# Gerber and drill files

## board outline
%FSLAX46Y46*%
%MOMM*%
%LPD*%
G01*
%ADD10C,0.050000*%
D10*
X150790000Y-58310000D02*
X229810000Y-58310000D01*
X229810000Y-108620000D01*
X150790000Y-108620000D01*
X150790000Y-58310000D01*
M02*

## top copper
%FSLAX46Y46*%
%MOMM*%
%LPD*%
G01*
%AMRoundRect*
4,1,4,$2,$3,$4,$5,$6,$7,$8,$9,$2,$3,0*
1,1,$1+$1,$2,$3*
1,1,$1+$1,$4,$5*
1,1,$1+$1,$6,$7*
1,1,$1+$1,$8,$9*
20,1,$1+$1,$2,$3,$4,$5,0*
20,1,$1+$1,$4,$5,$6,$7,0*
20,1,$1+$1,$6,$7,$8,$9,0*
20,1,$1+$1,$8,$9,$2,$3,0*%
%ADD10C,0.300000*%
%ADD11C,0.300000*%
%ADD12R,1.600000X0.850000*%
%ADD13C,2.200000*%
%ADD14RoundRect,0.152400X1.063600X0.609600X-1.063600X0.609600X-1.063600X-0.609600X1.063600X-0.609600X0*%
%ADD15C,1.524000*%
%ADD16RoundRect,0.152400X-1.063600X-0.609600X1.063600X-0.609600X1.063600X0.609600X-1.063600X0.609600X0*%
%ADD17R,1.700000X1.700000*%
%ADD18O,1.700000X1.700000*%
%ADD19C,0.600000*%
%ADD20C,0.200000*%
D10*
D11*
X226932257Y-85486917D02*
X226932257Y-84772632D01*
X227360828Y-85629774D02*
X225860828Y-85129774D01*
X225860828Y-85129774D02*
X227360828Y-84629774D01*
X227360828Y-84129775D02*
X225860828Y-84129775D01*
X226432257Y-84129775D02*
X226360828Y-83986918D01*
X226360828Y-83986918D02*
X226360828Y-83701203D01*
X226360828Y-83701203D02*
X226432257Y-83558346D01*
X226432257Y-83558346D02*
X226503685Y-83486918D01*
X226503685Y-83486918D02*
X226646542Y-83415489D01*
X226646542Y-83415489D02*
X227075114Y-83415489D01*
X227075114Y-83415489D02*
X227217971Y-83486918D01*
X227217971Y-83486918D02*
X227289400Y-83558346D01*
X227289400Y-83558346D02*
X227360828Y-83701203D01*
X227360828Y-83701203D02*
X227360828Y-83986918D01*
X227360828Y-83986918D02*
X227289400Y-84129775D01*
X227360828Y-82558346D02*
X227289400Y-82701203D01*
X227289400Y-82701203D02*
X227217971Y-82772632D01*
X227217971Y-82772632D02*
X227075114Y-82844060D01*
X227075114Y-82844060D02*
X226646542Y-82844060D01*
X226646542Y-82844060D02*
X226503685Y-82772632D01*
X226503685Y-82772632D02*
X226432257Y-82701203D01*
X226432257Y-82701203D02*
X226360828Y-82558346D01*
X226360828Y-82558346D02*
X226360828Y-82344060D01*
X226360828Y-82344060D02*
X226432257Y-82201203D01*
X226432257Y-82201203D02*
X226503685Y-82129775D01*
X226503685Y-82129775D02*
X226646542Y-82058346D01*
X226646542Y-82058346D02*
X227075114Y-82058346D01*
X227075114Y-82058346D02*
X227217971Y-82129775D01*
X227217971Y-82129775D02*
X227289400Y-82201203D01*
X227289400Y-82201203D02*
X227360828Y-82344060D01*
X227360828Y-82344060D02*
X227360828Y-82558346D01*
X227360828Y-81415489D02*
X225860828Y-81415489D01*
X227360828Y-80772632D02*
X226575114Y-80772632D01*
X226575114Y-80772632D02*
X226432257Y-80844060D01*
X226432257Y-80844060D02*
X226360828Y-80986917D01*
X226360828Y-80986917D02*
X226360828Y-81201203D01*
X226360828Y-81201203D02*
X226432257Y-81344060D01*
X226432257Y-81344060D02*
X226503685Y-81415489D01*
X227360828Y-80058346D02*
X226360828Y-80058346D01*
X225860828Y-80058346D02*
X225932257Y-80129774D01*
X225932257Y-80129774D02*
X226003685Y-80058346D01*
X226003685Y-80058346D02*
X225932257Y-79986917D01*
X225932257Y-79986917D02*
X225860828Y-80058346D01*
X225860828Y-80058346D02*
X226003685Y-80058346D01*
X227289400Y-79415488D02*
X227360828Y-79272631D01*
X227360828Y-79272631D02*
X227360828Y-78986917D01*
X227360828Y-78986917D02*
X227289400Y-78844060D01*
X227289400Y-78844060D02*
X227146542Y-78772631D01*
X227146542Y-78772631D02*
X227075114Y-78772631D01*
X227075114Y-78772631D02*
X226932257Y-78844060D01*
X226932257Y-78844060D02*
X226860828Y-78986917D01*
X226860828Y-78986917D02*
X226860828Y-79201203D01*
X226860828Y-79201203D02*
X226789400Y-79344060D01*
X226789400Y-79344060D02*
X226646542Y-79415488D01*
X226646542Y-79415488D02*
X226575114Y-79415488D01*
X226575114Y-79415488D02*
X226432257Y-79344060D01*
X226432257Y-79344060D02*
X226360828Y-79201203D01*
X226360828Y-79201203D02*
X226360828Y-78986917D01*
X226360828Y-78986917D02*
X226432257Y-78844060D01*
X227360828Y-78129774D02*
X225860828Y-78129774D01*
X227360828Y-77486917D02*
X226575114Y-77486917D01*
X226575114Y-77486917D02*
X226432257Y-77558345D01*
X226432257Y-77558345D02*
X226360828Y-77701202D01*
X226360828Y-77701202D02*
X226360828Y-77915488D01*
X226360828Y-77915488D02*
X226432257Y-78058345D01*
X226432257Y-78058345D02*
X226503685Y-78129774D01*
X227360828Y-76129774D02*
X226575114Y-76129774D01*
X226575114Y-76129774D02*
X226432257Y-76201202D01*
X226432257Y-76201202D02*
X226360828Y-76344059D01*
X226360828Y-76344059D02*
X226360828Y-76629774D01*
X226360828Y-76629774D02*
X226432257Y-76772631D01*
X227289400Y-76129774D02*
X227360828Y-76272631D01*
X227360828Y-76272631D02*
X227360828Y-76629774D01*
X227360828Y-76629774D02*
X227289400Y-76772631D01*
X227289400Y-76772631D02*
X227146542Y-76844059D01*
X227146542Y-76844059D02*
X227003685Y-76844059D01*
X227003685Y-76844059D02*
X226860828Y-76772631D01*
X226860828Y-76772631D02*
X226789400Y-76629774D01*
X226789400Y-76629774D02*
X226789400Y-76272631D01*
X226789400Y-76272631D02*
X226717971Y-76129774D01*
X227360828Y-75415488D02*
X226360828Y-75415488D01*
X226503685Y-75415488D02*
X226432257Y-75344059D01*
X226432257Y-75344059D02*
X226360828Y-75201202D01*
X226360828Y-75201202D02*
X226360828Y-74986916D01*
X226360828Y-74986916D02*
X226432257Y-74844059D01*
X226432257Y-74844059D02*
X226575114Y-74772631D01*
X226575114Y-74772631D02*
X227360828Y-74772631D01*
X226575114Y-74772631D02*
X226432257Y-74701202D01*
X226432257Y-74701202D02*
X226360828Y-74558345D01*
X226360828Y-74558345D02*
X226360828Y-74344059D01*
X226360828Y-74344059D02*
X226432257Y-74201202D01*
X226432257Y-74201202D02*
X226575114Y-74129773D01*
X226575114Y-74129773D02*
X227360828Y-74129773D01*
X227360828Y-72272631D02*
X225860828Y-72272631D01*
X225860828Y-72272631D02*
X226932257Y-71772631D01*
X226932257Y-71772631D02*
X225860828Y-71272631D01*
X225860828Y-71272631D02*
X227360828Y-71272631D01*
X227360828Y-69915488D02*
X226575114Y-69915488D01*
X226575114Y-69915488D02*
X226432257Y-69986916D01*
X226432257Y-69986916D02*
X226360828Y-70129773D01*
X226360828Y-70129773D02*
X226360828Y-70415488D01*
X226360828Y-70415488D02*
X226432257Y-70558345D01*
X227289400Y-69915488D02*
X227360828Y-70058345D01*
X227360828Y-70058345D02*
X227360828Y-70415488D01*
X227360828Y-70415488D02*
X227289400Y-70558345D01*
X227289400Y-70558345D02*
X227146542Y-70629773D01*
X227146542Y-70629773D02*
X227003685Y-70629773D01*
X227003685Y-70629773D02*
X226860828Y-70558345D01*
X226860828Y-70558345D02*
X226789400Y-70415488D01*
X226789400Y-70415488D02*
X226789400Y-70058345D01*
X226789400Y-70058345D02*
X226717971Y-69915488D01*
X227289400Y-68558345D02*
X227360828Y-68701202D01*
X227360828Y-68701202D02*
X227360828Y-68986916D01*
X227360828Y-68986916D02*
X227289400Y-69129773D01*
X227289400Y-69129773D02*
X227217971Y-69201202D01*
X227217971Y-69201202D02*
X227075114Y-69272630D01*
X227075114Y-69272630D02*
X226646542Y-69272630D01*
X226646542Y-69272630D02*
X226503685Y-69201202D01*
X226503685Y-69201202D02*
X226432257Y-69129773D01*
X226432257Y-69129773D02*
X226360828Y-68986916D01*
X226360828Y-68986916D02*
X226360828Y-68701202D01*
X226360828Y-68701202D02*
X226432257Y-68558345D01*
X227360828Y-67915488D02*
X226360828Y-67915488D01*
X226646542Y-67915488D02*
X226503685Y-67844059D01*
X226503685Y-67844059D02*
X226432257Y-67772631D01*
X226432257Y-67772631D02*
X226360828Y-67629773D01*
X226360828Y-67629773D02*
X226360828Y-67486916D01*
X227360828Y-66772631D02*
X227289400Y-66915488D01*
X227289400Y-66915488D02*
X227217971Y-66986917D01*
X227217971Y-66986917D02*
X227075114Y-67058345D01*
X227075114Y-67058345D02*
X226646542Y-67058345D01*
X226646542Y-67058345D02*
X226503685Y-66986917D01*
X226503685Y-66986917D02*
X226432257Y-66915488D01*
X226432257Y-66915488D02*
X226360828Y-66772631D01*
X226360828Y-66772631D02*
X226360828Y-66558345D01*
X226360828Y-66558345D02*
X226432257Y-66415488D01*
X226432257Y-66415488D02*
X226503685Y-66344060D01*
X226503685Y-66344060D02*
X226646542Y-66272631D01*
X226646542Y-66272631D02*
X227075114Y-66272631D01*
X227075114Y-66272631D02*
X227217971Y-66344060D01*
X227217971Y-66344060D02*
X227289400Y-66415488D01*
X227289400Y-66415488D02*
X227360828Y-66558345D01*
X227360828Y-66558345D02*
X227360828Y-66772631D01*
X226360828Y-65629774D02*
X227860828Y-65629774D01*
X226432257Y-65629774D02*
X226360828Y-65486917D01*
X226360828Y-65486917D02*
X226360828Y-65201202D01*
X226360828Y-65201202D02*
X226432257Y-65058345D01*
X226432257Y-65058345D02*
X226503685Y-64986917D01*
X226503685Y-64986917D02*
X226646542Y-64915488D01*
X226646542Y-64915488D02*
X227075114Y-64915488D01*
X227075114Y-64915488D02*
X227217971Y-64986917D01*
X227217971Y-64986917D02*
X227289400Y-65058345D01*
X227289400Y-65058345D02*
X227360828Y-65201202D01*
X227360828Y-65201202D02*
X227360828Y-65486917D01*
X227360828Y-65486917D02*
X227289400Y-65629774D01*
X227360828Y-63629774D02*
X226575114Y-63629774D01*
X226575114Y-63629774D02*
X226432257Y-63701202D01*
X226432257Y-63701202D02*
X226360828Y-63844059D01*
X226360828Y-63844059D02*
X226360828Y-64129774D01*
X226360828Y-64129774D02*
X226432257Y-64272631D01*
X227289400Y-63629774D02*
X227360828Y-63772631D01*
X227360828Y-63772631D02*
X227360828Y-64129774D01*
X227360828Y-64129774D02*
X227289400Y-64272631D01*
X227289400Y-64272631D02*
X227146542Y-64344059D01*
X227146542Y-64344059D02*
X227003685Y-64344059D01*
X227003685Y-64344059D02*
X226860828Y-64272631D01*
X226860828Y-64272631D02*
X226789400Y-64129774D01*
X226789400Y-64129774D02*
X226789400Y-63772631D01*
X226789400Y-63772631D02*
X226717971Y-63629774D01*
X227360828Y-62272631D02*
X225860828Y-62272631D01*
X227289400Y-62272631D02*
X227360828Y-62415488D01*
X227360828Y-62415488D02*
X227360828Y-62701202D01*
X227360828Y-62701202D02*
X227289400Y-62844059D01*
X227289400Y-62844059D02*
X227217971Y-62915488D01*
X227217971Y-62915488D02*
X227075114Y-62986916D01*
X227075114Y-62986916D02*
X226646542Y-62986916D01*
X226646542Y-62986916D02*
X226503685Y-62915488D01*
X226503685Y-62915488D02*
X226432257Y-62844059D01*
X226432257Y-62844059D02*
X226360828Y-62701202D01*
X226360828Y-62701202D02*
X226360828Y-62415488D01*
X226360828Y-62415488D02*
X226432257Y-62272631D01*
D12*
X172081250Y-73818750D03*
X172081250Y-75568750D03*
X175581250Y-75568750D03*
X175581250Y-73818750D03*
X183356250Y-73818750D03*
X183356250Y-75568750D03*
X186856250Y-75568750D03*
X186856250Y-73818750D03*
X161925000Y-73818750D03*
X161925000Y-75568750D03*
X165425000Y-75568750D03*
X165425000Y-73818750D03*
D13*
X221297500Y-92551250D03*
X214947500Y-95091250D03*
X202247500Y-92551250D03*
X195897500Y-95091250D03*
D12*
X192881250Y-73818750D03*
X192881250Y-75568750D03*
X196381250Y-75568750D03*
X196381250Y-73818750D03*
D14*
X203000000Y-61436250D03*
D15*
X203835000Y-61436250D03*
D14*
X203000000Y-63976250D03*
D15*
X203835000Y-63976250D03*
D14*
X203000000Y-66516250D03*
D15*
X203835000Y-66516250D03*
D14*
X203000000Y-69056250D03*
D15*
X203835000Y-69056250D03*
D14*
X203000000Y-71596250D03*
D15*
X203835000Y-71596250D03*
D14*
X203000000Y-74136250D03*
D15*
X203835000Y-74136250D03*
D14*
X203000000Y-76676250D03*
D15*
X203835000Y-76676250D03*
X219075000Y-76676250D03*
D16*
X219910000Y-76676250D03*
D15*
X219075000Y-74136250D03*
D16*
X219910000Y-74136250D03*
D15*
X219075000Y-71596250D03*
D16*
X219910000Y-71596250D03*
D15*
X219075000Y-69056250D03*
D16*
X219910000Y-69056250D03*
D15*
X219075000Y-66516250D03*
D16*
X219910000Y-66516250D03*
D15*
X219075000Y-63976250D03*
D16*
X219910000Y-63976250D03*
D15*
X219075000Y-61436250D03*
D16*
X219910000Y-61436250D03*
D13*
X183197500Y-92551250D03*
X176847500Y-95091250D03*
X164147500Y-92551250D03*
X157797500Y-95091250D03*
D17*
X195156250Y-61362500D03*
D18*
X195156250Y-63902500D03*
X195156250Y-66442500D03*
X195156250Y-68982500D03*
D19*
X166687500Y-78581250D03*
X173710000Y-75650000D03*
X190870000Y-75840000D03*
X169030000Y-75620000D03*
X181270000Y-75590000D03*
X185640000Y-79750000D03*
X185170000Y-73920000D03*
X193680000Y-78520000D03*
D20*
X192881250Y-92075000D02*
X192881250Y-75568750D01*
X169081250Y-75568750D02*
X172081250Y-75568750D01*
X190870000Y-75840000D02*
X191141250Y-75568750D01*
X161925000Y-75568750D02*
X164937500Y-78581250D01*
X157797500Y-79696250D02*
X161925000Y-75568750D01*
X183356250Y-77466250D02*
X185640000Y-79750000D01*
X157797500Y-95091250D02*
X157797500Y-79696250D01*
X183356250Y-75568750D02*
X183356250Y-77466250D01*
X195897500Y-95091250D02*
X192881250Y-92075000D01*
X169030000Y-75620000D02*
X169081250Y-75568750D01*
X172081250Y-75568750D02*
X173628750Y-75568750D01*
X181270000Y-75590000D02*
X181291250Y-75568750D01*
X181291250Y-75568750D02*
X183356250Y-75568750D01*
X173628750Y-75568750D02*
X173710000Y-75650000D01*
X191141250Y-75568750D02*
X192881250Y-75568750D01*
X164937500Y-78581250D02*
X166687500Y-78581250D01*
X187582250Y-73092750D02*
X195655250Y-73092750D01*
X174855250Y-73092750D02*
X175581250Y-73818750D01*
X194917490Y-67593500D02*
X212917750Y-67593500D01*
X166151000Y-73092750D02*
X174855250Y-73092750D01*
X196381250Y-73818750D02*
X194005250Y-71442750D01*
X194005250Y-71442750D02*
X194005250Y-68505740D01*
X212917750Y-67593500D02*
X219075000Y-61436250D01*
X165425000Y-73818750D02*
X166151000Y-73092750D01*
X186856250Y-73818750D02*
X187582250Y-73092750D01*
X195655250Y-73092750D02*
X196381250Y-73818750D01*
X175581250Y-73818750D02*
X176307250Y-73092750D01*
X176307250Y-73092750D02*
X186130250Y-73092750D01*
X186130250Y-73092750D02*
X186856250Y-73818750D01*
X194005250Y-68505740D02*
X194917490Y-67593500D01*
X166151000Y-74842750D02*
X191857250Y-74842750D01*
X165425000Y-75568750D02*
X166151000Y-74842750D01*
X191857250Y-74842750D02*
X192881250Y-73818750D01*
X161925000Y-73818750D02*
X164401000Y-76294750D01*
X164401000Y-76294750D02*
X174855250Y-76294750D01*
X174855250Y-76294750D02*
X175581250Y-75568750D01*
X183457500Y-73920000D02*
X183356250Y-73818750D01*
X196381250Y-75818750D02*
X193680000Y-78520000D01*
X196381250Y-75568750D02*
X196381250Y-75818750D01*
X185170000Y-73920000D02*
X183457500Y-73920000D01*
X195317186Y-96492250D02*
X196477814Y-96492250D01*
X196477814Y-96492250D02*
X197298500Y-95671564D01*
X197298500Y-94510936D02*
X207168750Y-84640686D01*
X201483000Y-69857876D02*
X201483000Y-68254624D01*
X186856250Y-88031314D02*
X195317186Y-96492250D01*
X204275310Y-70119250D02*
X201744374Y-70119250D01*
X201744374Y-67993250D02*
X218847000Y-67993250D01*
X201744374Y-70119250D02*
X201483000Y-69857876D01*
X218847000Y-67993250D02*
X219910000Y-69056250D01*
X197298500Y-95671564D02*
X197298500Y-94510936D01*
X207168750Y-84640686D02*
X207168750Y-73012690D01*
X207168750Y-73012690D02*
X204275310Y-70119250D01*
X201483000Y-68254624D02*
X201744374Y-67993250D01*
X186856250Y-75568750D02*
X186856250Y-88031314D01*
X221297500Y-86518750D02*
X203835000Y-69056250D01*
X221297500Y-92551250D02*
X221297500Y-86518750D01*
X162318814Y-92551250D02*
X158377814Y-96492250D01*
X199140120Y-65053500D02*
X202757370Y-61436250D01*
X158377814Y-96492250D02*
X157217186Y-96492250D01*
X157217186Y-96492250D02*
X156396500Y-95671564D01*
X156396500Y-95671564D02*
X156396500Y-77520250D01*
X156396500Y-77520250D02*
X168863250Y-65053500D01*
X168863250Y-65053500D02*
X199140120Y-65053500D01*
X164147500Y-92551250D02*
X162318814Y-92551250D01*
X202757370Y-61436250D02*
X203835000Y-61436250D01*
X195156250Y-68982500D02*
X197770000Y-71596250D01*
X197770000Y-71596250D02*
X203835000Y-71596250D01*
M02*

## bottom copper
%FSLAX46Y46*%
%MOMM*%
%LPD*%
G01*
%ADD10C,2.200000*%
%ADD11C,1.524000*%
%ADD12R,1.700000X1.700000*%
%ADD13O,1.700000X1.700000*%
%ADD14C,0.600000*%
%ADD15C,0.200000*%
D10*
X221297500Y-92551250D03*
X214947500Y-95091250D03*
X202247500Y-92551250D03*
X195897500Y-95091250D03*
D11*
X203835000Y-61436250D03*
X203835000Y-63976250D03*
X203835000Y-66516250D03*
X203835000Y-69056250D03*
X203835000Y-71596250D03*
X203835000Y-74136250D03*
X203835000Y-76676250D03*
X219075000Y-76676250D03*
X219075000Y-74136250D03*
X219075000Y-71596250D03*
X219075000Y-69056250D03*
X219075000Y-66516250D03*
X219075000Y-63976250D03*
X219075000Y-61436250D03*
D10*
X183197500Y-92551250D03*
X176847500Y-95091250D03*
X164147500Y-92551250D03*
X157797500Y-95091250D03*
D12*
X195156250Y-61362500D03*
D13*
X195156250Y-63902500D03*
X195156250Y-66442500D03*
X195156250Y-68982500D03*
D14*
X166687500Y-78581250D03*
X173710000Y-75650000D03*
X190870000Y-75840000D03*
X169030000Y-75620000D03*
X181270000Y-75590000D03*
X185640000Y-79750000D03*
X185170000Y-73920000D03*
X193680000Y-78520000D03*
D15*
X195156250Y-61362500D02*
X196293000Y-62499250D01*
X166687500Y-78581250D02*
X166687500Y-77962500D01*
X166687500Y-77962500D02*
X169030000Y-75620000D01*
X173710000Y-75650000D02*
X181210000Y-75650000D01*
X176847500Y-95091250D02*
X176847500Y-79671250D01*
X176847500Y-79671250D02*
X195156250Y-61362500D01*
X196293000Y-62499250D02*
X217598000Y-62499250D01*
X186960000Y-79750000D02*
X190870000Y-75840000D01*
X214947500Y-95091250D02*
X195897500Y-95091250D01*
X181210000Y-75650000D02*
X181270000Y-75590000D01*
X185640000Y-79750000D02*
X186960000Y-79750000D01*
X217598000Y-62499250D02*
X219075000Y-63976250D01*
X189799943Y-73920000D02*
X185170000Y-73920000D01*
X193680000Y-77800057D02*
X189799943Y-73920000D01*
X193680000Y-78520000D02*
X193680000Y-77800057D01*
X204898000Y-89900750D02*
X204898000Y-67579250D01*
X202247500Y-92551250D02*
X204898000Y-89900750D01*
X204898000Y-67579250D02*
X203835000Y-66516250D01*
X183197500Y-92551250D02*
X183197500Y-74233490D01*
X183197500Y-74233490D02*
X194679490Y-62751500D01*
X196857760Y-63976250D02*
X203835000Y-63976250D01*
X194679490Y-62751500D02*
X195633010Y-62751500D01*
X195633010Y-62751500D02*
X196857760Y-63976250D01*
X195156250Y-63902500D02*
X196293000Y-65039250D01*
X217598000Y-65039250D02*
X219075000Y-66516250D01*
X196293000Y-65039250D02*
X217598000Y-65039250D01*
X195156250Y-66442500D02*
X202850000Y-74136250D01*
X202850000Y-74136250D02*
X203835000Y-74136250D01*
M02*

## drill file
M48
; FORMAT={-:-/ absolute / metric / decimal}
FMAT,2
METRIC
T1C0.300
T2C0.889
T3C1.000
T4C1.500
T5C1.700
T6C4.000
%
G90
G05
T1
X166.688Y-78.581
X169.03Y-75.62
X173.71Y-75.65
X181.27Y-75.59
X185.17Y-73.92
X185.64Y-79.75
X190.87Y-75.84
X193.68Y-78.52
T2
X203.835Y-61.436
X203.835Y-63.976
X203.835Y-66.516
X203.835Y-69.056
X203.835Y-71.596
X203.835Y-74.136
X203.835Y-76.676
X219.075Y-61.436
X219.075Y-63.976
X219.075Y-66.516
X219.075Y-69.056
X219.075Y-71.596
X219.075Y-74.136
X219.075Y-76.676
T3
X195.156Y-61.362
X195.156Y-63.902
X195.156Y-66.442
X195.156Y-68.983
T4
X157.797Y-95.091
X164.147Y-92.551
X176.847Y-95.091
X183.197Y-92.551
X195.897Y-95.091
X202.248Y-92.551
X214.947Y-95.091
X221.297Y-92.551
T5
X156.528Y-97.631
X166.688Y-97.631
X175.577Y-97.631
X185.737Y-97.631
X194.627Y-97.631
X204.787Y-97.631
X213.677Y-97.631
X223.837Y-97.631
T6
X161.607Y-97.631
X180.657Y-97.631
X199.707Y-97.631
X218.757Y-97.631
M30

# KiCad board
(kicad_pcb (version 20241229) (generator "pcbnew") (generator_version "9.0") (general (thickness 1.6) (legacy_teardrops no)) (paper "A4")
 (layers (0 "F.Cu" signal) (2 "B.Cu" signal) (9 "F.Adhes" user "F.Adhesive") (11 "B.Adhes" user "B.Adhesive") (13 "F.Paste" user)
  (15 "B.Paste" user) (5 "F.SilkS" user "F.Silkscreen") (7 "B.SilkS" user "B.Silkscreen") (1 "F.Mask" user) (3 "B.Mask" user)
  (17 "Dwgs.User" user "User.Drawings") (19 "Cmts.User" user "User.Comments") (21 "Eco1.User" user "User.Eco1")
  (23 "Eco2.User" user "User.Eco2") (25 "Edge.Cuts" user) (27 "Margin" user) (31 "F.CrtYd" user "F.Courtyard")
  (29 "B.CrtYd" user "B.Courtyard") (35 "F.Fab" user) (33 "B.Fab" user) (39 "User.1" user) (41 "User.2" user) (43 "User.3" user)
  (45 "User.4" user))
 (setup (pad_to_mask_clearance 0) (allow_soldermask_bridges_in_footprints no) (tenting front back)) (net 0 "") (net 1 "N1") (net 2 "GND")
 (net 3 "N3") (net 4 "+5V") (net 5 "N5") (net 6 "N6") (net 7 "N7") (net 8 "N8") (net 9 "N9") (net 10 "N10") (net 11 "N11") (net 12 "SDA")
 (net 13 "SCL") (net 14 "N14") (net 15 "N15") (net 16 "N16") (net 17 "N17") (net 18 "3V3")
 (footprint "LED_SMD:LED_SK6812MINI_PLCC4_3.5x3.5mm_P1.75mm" (layer "F.Cu") (at 173.83125 74.69375)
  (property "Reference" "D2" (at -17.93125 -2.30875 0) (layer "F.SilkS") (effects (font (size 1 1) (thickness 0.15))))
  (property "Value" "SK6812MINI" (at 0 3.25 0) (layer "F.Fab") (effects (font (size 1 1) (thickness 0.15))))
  (pad "1" smd rect (at -1.75 -0.875) (size 1.6 0.85) (layers "F.Cu" "F.Mask" "F.Paste") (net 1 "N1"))
  (pad "2" smd rect (at -1.75 0.875) (size 1.6 0.85) (layers "F.Cu" "F.Mask" "F.Paste") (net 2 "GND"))
  (pad "3" smd rect (at 1.75 0.875) (size 1.6 0.85) (layers "F.Cu" "F.Mask" "F.Paste") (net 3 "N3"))
  (pad "4" smd rect (at 1.75 -0.875) (size 1.6 0.85) (layers "F.Cu" "F.Mask" "F.Paste") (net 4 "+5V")))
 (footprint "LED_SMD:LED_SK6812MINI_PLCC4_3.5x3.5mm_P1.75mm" (layer "F.Cu") (at 185.10625 74.69375)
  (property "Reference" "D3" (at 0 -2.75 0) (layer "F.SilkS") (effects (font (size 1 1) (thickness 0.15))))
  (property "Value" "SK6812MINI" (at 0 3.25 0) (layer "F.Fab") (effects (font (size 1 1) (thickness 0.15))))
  (pad "1" smd rect (at -1.75 -0.875) (size 1.6 0.85) (layers "F.Cu" "F.Mask" "F.Paste") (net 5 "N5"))
  (pad "2" smd rect (at -1.75 0.875) (size 1.6 0.85) (layers "F.Cu" "F.Mask" "F.Paste") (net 2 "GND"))
  (pad "3" smd rect (at 1.75 0.875) (size 1.6 0.85) (layers "F.Cu" "F.Mask" "F.Paste") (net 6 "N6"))
  (pad "4" smd rect (at 1.75 -0.875) (size 1.6 0.85) (layers "F.Cu" "F.Mask" "F.Paste") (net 4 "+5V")))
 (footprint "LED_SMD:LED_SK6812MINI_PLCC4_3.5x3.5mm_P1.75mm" (layer "F.Cu") (at 163.675 74.69375)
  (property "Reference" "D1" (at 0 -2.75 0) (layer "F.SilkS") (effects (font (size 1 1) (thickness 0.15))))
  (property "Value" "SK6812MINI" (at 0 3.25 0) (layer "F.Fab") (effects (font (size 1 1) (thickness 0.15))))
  (pad "1" smd rect (at -1.75 -0.875) (size 1.6 0.85) (layers "F.Cu" "F.Mask" "F.Paste") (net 3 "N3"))
  (pad "2" smd rect (at -1.75 0.875) (size 1.6 0.85) (layers "F.Cu" "F.Mask" "F.Paste") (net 2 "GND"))
  (pad "3" smd rect (at 1.75 0.875) (size 1.6 0.85) (layers "F.Cu" "F.Mask" "F.Paste") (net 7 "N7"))
  (pad "4" smd rect (at 1.75 -0.875) (size 1.6 0.85) (layers "F.Cu" "F.Mask" "F.Paste") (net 4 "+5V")))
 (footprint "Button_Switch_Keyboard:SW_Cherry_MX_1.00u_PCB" (layer "F.Cu") (at 221.2975 92.55125)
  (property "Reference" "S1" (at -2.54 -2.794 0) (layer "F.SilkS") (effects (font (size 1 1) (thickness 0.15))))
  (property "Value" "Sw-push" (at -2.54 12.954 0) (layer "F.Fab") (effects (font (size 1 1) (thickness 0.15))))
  (pad "" np_thru_hole circle (at -7.62 5.08) (size 1.7 1.7) (drill 1.7) (layers "*.Cu" "*.Mask"))
  (pad "" np_thru_hole circle (at -2.54 5.08) (size 4 4) (drill 4) (layers "*.Cu" "*.Mask"))
  (pad "" np_thru_hole circle (at 2.54 5.08) (size 1.7 1.7) (drill 1.7) (layers "*.Cu" "*.Mask"))
  (pad "1" thru_hole circle (at 0 0) (size 2.2 2.2) (drill 1.5) (layers "*.Cu" "*.Mask") (remove_unused_layers no) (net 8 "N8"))
  (pad "2" thru_hole circle (at -6.35 2.54) (size 2.2 2.2) (drill 1.5) (layers "*.Cu" "*.Mask") (remove_unused_layers no) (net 2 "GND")))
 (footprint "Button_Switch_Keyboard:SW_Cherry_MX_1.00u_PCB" (layer "F.Cu") (at 202.2475 92.55125)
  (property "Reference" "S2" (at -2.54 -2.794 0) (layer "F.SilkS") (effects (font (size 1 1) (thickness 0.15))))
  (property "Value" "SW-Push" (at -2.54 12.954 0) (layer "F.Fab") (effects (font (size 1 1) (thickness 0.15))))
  (pad "" np_thru_hole circle (at -7.62 5.08) (size 1.7 1.7) (drill 1.7) (layers "*.Cu" "*.Mask"))
  (pad "" np_thru_hole circle (at -2.54 5.08) (size 4 4) (drill 4) (layers "*.Cu" "*.Mask"))
  (pad "" np_thru_hole circle (at 2.54 5.08) (size 1.7 1.7) (drill 1.7) (layers "*.Cu" "*.Mask"))
  (pad "1" thru_hole circle (at 0 0) (size 2.2 2.2) (drill 1.5) (layers "*.Cu" "*.Mask") (remove_unused_layers no) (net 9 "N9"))
  (pad "2" thru_hole circle (at -6.35 2.54) (size 2.2 2.2) (drill 1.5) (layers "*.Cu" "*.Mask") (remove_unused_layers no) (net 2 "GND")))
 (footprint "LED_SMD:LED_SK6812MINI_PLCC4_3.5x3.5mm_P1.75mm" (layer "F.Cu") (at 194.63125 74.69375)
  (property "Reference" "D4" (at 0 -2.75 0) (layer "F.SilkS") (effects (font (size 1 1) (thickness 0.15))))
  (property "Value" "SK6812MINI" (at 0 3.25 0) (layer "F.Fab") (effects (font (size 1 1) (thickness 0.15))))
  (pad "1" smd rect (at -1.75 -0.875) (size 1.6 0.85) (layers "F.Cu" "F.Mask" "F.Paste") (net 7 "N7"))
  (pad "2" smd rect (at -1.75 0.875) (size 1.6 0.85) (layers "F.Cu" "F.Mask" "F.Paste") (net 2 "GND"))
  (pad "3" smd rect (at 1.75 0.875) (size 1.6 0.85) (layers "F.Cu" "F.Mask" "F.Paste") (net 5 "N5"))
  (pad "4" smd rect (at 1.75 -0.875) (size 1.6 0.85) (layers "F.Cu" "F.Mask" "F.Paste") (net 4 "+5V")))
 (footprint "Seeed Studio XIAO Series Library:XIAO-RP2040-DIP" (layer "F.Cu") (at 211.455 69.05625)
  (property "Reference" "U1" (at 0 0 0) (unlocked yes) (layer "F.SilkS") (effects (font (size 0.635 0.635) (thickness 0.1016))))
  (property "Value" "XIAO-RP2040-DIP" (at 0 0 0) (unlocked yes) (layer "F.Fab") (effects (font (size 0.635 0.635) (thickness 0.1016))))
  (pad "1" smd roundrect (at -8.455 -7.62 180) (size 2.432 1.524) (layers "F.Cu" "F.Mask") (roundrect_rratio 0.1) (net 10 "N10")
   (thermal_bridge_angle 45))
  (pad "1" thru_hole circle (at -7.62 -7.62 180) (size 1.524 1.524) (drill 0.889) (layers "*.Cu" "*.Mask") (remove_unused_layers no)
   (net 10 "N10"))
  (pad "2" smd roundrect (at -8.455 -5.08 180) (size 2.432 1.524) (layers "F.Cu" "F.Mask") (roundrect_rratio 0.1) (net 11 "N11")
   (thermal_bridge_angle 45))
  (pad "2" thru_hole circle (at -7.62 -5.08 180) (size 1.524 1.524) (drill 0.889) (layers "*.Cu" "*.Mask") (remove_unused_layers no)
   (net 11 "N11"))
  (pad "3" smd roundrect (at -8.455 -2.54 180) (size 2.432 1.524) (layers "F.Cu" "F.Mask") (roundrect_rratio 0.1) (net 9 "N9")
   (thermal_bridge_angle 45))
  (pad "3" thru_hole circle (at -7.62 -2.54 180) (size 1.524 1.524) (drill 0.889) (layers "*.Cu" "*.Mask") (remove_unused_layers no)
   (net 9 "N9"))
  (pad "4" smd roundrect (at -8.455 0 180) (size 2.432 1.524) (layers "F.Cu" "F.Mask") (roundrect_rratio 0.1) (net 8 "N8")
   (thermal_bridge_angle 45))
  (pad "4" thru_hole circle (at -7.62 0 180) (size 1.524 1.524) (drill 0.889) (layers "*.Cu" "*.Mask") (remove_unused_layers no)
   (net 8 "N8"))
  (pad "5" smd roundrect (at -8.455 2.54 180) (size 2.432 1.524) (layers "F.Cu" "F.Mask") (roundrect_rratio 0.1) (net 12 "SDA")
   (thermal_bridge_angle 45))
  (pad "5" thru_hole circle (at -7.62 2.54 180) (size 1.524 1.524) (drill 0.889) (layers "*.Cu" "*.Mask") (remove_unused_layers no)
   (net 12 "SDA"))
  (pad "6" smd roundrect (at -8.455 5.08 180) (size 2.432 1.524) (layers "F.Cu" "F.Mask") (roundrect_rratio 0.1) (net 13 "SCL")
   (thermal_bridge_angle 45))
  (pad "6" thru_hole circle (at -7.62 5.08 180) (size 1.524 1.524) (drill 0.889) (layers "*.Cu" "*.Mask") (remove_unused_layers no)
   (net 13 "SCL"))
  (pad "7" smd roundrect (at -8.455 7.62 180) (size 2.432 1.524) (layers "F.Cu" "F.Mask") (roundrect_rratio 0.1) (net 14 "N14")
   (thermal_bridge_angle 45))
  (pad "7" thru_hole circle (at -7.62 7.62 180) (size 1.524 1.524) (drill 0.889) (layers "*.Cu" "*.Mask") (remove_unused_layers no)
   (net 14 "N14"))
  (pad "8" thru_hole circle (at 7.62 7.62) (size 1.524 1.524) (drill 0.889) (layers "*.Cu" "*.Mask") (remove_unused_layers no)
   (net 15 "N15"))
  (pad "8" smd roundrect (at 8.455 7.62) (size 2.432 1.524) (layers "F.Cu" "F.Mask") (roundrect_rratio 0.1) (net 15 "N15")
   (thermal_bridge_angle 45))
  (pad "9" thru_hole circle (at 7.62 5.08) (size 1.524 1.524) (drill 0.889) (layers "*.Cu" "*.Mask") (remove_unused_layers no)
   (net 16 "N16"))
  (pad "9" smd roundrect (at 8.455 5.08) (size 2.432 1.524) (layers "F.Cu" "F.Mask") (roundrect_rratio 0.1) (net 16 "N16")
   (thermal_bridge_angle 45))
  (pad "10" thru_hole circle (at 7.62 2.54) (size 1.524 1.524) (drill 0.889) (layers "*.Cu" "*.Mask") (remove_unused_layers no)
   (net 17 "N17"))
  (pad "10" smd roundrect (at 8.455 2.54) (size 2.432 1.524) (layers "F.Cu" "F.Mask") (roundrect_rratio 0.1) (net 17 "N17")
   (thermal_bridge_angle 45))
  (pad "11" thru_hole circle (at 7.62 0) (size 1.524 1.524) (drill 0.889) (layers "*.Cu" "*.Mask") (remove_unused_layers no) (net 6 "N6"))
  (pad "11" smd roundrect (at 8.455 0) (size 2.432 1.524) (layers "F.Cu" "F.Mask") (roundrect_rratio 0.1) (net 6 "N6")
   (thermal_bridge_angle 45))
  (pad "12" thru_hole circle (at 7.62 -2.54) (size 1.524 1.524) (drill 0.889) (layers "*.Cu" "*.Mask") (remove_unused_layers no)
   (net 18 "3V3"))
  (pad "12" smd roundrect (at 8.455 -2.54) (size 2.432 1.524) (layers "F.Cu" "F.Mask") (roundrect_rratio 0.1) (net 18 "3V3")
   (thermal_bridge_angle 45))
  (pad "13" thru_hole circle (at 7.62 -5.08) (size 1.524 1.524) (drill 0.889) (layers "*.Cu" "*.Mask") (remove_unused_layers no)
   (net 2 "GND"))
  (pad "13" smd roundrect (at 8.455 -5.08) (size 2.432 1.524) (layers "F.Cu" "F.Mask") (roundrect_rratio 0.1) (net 2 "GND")
   (thermal_bridge_angle 45))
  (pad "14" thru_hole circle (at 7.62 -7.62) (size 1.524 1.524) (drill 0.889) (layers "*.Cu" "*.Mask") (remove_unused_layers no)
   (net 4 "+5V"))
  (pad "14" smd roundrect (at 8.455 -7.62) (size 2.432 1.524) (layers "F.Cu" "F.Mask") (roundrect_rratio 0.1) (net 4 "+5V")
   (thermal_bridge_angle 45)))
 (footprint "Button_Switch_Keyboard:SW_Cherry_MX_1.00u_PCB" (layer "F.Cu") (at 183.1975 92.55125)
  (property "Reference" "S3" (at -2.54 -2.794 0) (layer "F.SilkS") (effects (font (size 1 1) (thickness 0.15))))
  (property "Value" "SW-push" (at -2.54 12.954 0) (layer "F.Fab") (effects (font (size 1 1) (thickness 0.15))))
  (pad "" np_thru_hole circle (at -7.62 5.08) (size 1.7 1.7) (drill 1.7) (layers "*.Cu" "*.Mask"))
  (pad "" np_thru_hole circle (at -2.54 5.08) (size 4 4) (drill 4) (layers "*.Cu" "*.Mask"))
  (pad "" np_thru_hole circle (at 2.54 5.08) (size 1.7 1.7) (drill 1.7) (layers "*.Cu" "*.Mask"))
  (pad "1" thru_hole circle (at 0 0) (size 2.2 2.2) (drill 1.5) (layers "*.Cu" "*.Mask") (remove_unused_layers no) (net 11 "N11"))
  (pad "2" thru_hole circle (at -6.35 2.54) (size 2.2 2.2) (drill 1.5) (layers "*.Cu" "*.Mask") (remove_unused_layers no) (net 2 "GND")))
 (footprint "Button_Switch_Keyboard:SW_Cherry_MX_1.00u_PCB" (layer "F.Cu") (at 164.1475 92.55125)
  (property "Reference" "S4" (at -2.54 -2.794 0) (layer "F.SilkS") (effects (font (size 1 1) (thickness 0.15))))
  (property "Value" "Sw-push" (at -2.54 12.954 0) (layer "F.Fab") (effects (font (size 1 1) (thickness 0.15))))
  (pad "" np_thru_hole circle (at -7.62 5.08) (size 1.7 1.7) (drill 1.7) (layers "*.Cu" "*.Mask"))
  (pad "" np_thru_hole circle (at -2.54 5.08) (size 4 4) (drill 4) (layers "*.Cu" "*.Mask"))
  (pad "" np_thru_hole circle (at 2.54 5.08) (size 1.7 1.7) (drill 1.7) (layers "*.Cu" "*.Mask"))
  (pad "1" thru_hole circle (at 0 0) (size 2.2 2.2) (drill 1.5) (layers "*.Cu" "*.Mask") (remove_unused_layers no) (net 10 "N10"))
  (pad "2" thru_hole circle (at -6.35 2.54) (size 2.2 2.2) (drill 1.5) (layers "*.Cu" "*.Mask") (remove_unused_layers no) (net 2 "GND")))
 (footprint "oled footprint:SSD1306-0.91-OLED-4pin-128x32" (layer "F.Cu") (at 158.65625 59.1725)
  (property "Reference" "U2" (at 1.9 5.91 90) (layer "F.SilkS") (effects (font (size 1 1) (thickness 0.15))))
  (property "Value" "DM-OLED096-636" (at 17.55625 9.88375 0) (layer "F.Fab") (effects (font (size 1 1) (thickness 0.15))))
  (pad "1" thru_hole rect (at 36.5 2.19) (size 1.7 1.7) (drill 1) (layers "*.Cu" "*.Mask") (remove_unused_layers no) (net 2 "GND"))
  (pad "2" thru_hole oval (at 36.5 4.73) (size 1.7 1.7) (drill 1) (layers "*.Cu" "*.Mask") (remove_unused_layers no) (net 18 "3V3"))
  (pad "3" thru_hole oval (at 36.5 7.27) (size 1.7 1.7) (drill 1) (layers "*.Cu" "*.Mask") (remove_unused_layers no) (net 13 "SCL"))
  (pad "4" thru_hole oval (at 36.5 9.81) (size 1.7 1.7) (drill 1) (layers "*.Cu" "*.Mask") (remove_unused_layers no) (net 12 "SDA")))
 (gr_rect (start 150.79 58.31) (end 229.81 108.62) (stroke (width 0.05) (type default)) (fill no) (layer "Edge.Cuts"))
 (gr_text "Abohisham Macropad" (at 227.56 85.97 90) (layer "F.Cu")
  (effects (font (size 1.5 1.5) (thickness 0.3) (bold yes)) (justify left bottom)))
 (segment (start 192.88125 92.075) (end 192.88125 75.56875) (width 0.2) (layer "F.Cu") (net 2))
 (segment (start 169.08125 75.56875) (end 172.08125 75.56875) (width 0.2) (layer "F.Cu") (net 2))
 (segment (start 190.87 75.84) (end 191.14125 75.56875) (width 0.2) (layer "F.Cu") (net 2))
 (segment (start 161.925 75.56875) (end 164.9375 78.58125) (width 0.2) (layer "F.Cu") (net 2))
 (segment (start 157.7975 79.69625) (end 161.925 75.56875) (width 0.2) (layer "F.Cu") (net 2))
 (segment (start 183.35625 77.46625) (end 185.64 79.75) (width 0.2) (layer "F.Cu") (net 2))
 (segment (start 157.7975 95.09125) (end 157.7975 79.69625) (width 0.2) (layer "F.Cu") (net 2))
 (segment (start 183.35625 75.56875) (end 183.35625 77.46625) (width 0.2) (layer "F.Cu") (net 2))
 (segment (start 195.8975 95.09125) (end 192.88125 92.075) (width 0.2) (layer "F.Cu") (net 2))
 (segment (start 169.03 75.62) (end 169.08125 75.56875) (width 0.2) (layer "F.Cu") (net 2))
 (segment (start 172.08125 75.56875) (end 173.62875 75.56875) (width 0.2) (layer "F.Cu") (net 2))
 (segment (start 181.27 75.59) (end 181.29125 75.56875) (width 0.2) (layer "F.Cu") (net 2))
 (segment (start 181.29125 75.56875) (end 183.35625 75.56875) (width 0.2) (layer "F.Cu") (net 2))
 (segment (start 173.62875 75.56875) (end 173.71 75.65) (width 0.2) (layer "F.Cu") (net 2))
 (segment (start 191.14125 75.56875) (end 192.88125 75.56875) (width 0.2) (layer "F.Cu") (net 2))
 (segment (start 164.9375 78.58125) (end 166.6875 78.58125) (width 0.2) (layer "F.Cu") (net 2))
 (via (at 166.6875 78.58125) (size 0.6) (drill 0.3) (layers "F.Cu" "B.Cu") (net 2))
 (via (at 173.71 75.65) (size 0.6) (drill 0.3) (layers "F.Cu" "B.Cu") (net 2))
 (via (at 190.87 75.84) (size 0.6) (drill 0.3) (layers "F.Cu" "B.Cu") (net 2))
 (via (at 169.03 75.62) (size 0.6) (drill 0.3) (layers "F.Cu" "B.Cu") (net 2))
 (via (at 181.27 75.59) (size 0.6) (drill 0.3) (layers "F.Cu" "B.Cu") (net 2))
 (via (at 185.64 79.75) (size 0.6) (drill 0.3) (layers "F.Cu" "B.Cu") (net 2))
 (segment (start 195.15625 61.3625) (end 196.293 62.49925) (width 0.2) (layer "B.Cu") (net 2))
 (segment (start 166.6875 78.58125) (end 166.6875 77.9625) (width 0.2) (layer "B.Cu") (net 2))
 (segment (start 166.6875 77.9625) (end 169.03 75.62) (width 0.2) (layer "B.Cu") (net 2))
 (segment (start 173.71 75.65) (end 181.21 75.65) (width 0.2) (layer "B.Cu") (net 2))
 (segment (start 176.8475 95.09125) (end 176.8475 79.67125) (width 0.2) (layer "B.Cu") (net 2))
 (segment (start 176.8475 79.67125) (end 195.15625 61.3625) (width 0.2) (layer "B.Cu") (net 2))
 (segment (start 196.293 62.49925) (end 217.598 62.49925) (width 0.2) (layer "B.Cu") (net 2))
 (segment (start 186.96 79.75) (end 190.87 75.84) (width 0.2) (layer "B.Cu") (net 2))
 (segment (start 214.9475 95.09125) (end 195.8975 95.09125) (width 0.2) (layer "B.Cu") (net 2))
 (segment (start 181.21 75.65) (end 181.27 75.59) (width 0.2) (layer "B.Cu") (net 2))
 (segment (start 185.64 79.75) (end 186.96 79.75) (width 0.2) (layer "B.Cu") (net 2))
 (segment (start 217.598 62.49925) (end 219.075 63.97625) (width 0.2) (layer "B.Cu") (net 2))
 (segment (start 187.58225 73.09275) (end 195.65525 73.09275) (width 0.2) (layer "F.Cu") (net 4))
 (segment (start 174.85525 73.09275) (end 175.58125 73.81875) (width 0.2) (layer "F.Cu") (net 4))
 (segment (start 194.91749 67.5935) (end 212.91775 67.5935) (width 0.2) (layer "F.Cu") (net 4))
 (segment (start 166.151 73.09275) (end 174.85525 73.09275) (width 0.2) (layer "F.Cu") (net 4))
 (segment (start 196.38125 73.81875) (end 194.00525 71.44275) (width 0.2) (layer "F.Cu") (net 4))
 (segment (start 194.00525 71.44275) (end 194.00525 68.50574) (width 0.2) (layer "F.Cu") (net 4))
 (segment (start 212.91775 67.5935) (end 219.075 61.43625) (width 0.2) (layer "F.Cu") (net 4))
 (segment (start 165.425 73.81875) (end 166.151 73.09275) (width 0.2) (layer "F.Cu") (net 4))
 (segment (start 186.85625 73.81875) (end 187.58225 73.09275) (width 0.2) (layer "F.Cu") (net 4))
 (segment (start 195.65525 73.09275) (end 196.38125 73.81875) (width 0.2) (layer "F.Cu") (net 4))
 (segment (start 175.58125 73.81875) (end 176.30725 73.09275) (width 0.2) (layer "F.Cu") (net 4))
 (segment (start 176.30725 73.09275) (end 186.13025 73.09275) (width 0.2) (layer "F.Cu") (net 4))
 (segment (start 186.13025 73.09275) (end 186.85625 73.81875) (width 0.2) (layer "F.Cu") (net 4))
 (segment (start 194.00525 68.50574) (end 194.91749 67.5935) (width 0.2) (layer "F.Cu") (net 4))
 (segment (start 166.151 74.84275) (end 191.85725 74.84275) (width 0.2) (layer "F.Cu") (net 7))
 (segment (start 165.425 75.56875) (end 166.151 74.84275) (width 0.2) (layer "F.Cu") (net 7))
 (segment (start 191.85725 74.84275) (end 192.88125 73.81875) (width 0.2) (layer "F.Cu") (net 7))
 (segment (start 161.925 73.81875) (end 164.401 76.29475) (width 0.2) (layer "F.Cu") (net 3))
 (segment (start 164.401 76.29475) (end 174.85525 76.29475) (width 0.2) (layer "F.Cu") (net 3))
 (segment (start 174.85525 76.29475) (end 175.58125 75.56875) (width 0.2) (layer "F.Cu") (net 3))
 (segment (start 183.4575 73.92) (end 183.35625 73.81875) (width 0.2) (layer "F.Cu") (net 5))
 (segment (start 196.38125 75.81875) (end 193.68 78.52) (width 0.2) (layer "F.Cu") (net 5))
 (segment (start 196.38125 75.56875) (end 196.38125 75.81875) (width 0.2) (layer "F.Cu") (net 5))
 (segment (start 185.17 73.92) (end 183.4575 73.92) (width 0.2) (layer "F.Cu") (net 5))
 (via (at 185.17 73.92) (size 0.6) (drill 0.3) (layers "F.Cu" "B.Cu") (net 5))
 (via (at 193.68 78.52) (size 0.6) (drill 0.3) (layers "F.Cu" "B.Cu") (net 5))
 (segment (start 189.799943 73.92) (end 185.17 73.92) (width 0.2) (layer "B.Cu") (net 5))
 (segment (start 193.68 77.800057) (end 189.799943 73.92) (width 0.2) (layer "B.Cu") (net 5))
 (segment (start 193.68 78.52) (end 193.68 77.800057) (width 0.2) (layer "B.Cu") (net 5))
 (segment (start 195.317186 96.49225) (end 196.477814 96.49225) (width 0.2) (layer "F.Cu") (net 6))
 (segment (start 196.477814 96.49225) (end 197.2985 95.671564) (width 0.2) (layer "F.Cu") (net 6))
 (segment (start 197.2985 94.510936) (end 207.16875 84.640686) (width 0.2) (layer "F.Cu") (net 6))
 (segment (start 201.483 69.857876) (end 201.483 68.254624) (width 0.2) (layer "F.Cu") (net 6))
 (segment (start 186.85625 88.031314) (end 195.317186 96.49225) (width 0.2) (layer "F.Cu") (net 6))
 (segment (start 204.27531 70.11925) (end 201.744374 70.11925) (width 0.2) (layer "F.Cu") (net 6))
 (segment (start 201.744374 67.99325) (end 218.847 67.99325) (width 0.2) (layer "F.Cu") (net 6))
 (segment (start 201.744374 70.11925) (end 201.483 69.857876) (width 0.2) (layer "F.Cu") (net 6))
 (segment (start 218.847 67.99325) (end 219.91 69.05625) (width 0.2) (layer "F.Cu") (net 6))
 (segment (start 197.2985 95.671564) (end 197.2985 94.510936) (width 0.2) (layer "F.Cu") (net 6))
 (segment (start 207.16875 84.640686) (end 207.16875 73.01269) (width 0.2) (layer "F.Cu") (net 6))
 (segment (start 207.16875 73.01269) (end 204.27531 70.11925) (width 0.2) (layer "F.Cu") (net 6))
 (segment (start 201.483 68.254624) (end 201.744374 67.99325) (width 0.2) (layer "F.Cu") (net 6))
 (segment (start 186.85625 75.56875) (end 186.85625 88.031314) (width 0.2) (layer "F.Cu") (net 6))
 (segment (start 221.2975 86.51875) (end 203.835 69.05625) (width 0.2) (layer "F.Cu") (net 8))
 (segment (start 221.2975 92.55125) (end 221.2975 86.51875) (width 0.2) (layer "F.Cu") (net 8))
 (segment (start 204.898 89.90075) (end 204.898 67.57925) (width 0.2) (layer "B.Cu") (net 9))
 (segment (start 202.2475 92.55125) (end 204.898 89.90075) (width 0.2) (layer "B.Cu") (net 9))
 (segment (start 204.898 67.57925) (end 203.835 66.51625) (width 0.2) (layer "B.Cu") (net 9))
 (segment (start 183.1975 92.55125) (end 183.1975 74.23349) (width 0.2) (layer "B.Cu") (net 11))
 (segment (start 183.1975 74.23349) (end 194.67949 62.7515) (width 0.2) (layer "B.Cu") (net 11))
 (segment (start 196.85776 63.97625) (end 203.835 63.97625) (width 0.2) (layer "B.Cu") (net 11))
 (segment (start 194.67949 62.7515) (end 195.63301 62.7515) (width 0.2) (layer "B.Cu") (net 11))
 (segment (start 195.63301 62.7515) (end 196.85776 63.97625) (width 0.2) (layer "B.Cu") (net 11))
 (segment (start 162.318814 92.55125) (end 158.377814 96.49225) (width 0.2) (layer "F.Cu") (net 10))
 (segment (start 199.14012 65.0535) (end 202.75737 61.43625) (width 0.2) (layer "F.Cu") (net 10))
 (segment (start 158.377814 96.49225) (end 157.217186 96.49225) (width 0.2) (layer "F.Cu") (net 10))
 (segment (start 157.217186 96.49225) (end 156.3965 95.671564) (width 0.2) (layer "F.Cu") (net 10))
 (segment (start 156.3965 95.671564) (end 156.3965 77.52025) (width 0.2) (layer "F.Cu") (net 10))
 (segment (start 156.3965 77.52025) (end 168.86325 65.0535) (width 0.2) (layer "F.Cu") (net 10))
 (segment (start 168.86325 65.0535) (end 199.14012 65.0535) (width 0.2) (layer "F.Cu") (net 10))
 (segment (start 164.1475 92.55125) (end 162.318814 92.55125) (width 0.2) (layer "F.Cu") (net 10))
 (segment (start 202.75737 61.43625) (end 203.835 61.43625) (width 0.2) (layer "F.Cu") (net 10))
 (segment (start 195.15625 68.9825) (end 197.77 71.59625) (width 0.2) (layer "F.Cu") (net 12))
 (segment (start 197.77 71.59625) (end 203.835 71.59625) (width 0.2) (layer "F.Cu") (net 12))
 (segment (start 195.15625 63.9025) (end 196.293 65.03925) (width 0.2) (layer "B.Cu") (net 18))
 (segment (start 217.598 65.03925) (end 219.075 66.51625) (width 0.2) (layer "B.Cu") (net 18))
 (segment (start 196.293 65.03925) (end 217.598 65.03925) (width 0.2) (layer "B.Cu") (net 18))
 (segment (start 195.15625 66.4425) (end 202.85 74.13625) (width 0.2) (layer "B.Cu") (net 13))
 (segment (start 202.85 74.13625) (end 203.835 74.13625) (width 0.2) (layer "B.Cu") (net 13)))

